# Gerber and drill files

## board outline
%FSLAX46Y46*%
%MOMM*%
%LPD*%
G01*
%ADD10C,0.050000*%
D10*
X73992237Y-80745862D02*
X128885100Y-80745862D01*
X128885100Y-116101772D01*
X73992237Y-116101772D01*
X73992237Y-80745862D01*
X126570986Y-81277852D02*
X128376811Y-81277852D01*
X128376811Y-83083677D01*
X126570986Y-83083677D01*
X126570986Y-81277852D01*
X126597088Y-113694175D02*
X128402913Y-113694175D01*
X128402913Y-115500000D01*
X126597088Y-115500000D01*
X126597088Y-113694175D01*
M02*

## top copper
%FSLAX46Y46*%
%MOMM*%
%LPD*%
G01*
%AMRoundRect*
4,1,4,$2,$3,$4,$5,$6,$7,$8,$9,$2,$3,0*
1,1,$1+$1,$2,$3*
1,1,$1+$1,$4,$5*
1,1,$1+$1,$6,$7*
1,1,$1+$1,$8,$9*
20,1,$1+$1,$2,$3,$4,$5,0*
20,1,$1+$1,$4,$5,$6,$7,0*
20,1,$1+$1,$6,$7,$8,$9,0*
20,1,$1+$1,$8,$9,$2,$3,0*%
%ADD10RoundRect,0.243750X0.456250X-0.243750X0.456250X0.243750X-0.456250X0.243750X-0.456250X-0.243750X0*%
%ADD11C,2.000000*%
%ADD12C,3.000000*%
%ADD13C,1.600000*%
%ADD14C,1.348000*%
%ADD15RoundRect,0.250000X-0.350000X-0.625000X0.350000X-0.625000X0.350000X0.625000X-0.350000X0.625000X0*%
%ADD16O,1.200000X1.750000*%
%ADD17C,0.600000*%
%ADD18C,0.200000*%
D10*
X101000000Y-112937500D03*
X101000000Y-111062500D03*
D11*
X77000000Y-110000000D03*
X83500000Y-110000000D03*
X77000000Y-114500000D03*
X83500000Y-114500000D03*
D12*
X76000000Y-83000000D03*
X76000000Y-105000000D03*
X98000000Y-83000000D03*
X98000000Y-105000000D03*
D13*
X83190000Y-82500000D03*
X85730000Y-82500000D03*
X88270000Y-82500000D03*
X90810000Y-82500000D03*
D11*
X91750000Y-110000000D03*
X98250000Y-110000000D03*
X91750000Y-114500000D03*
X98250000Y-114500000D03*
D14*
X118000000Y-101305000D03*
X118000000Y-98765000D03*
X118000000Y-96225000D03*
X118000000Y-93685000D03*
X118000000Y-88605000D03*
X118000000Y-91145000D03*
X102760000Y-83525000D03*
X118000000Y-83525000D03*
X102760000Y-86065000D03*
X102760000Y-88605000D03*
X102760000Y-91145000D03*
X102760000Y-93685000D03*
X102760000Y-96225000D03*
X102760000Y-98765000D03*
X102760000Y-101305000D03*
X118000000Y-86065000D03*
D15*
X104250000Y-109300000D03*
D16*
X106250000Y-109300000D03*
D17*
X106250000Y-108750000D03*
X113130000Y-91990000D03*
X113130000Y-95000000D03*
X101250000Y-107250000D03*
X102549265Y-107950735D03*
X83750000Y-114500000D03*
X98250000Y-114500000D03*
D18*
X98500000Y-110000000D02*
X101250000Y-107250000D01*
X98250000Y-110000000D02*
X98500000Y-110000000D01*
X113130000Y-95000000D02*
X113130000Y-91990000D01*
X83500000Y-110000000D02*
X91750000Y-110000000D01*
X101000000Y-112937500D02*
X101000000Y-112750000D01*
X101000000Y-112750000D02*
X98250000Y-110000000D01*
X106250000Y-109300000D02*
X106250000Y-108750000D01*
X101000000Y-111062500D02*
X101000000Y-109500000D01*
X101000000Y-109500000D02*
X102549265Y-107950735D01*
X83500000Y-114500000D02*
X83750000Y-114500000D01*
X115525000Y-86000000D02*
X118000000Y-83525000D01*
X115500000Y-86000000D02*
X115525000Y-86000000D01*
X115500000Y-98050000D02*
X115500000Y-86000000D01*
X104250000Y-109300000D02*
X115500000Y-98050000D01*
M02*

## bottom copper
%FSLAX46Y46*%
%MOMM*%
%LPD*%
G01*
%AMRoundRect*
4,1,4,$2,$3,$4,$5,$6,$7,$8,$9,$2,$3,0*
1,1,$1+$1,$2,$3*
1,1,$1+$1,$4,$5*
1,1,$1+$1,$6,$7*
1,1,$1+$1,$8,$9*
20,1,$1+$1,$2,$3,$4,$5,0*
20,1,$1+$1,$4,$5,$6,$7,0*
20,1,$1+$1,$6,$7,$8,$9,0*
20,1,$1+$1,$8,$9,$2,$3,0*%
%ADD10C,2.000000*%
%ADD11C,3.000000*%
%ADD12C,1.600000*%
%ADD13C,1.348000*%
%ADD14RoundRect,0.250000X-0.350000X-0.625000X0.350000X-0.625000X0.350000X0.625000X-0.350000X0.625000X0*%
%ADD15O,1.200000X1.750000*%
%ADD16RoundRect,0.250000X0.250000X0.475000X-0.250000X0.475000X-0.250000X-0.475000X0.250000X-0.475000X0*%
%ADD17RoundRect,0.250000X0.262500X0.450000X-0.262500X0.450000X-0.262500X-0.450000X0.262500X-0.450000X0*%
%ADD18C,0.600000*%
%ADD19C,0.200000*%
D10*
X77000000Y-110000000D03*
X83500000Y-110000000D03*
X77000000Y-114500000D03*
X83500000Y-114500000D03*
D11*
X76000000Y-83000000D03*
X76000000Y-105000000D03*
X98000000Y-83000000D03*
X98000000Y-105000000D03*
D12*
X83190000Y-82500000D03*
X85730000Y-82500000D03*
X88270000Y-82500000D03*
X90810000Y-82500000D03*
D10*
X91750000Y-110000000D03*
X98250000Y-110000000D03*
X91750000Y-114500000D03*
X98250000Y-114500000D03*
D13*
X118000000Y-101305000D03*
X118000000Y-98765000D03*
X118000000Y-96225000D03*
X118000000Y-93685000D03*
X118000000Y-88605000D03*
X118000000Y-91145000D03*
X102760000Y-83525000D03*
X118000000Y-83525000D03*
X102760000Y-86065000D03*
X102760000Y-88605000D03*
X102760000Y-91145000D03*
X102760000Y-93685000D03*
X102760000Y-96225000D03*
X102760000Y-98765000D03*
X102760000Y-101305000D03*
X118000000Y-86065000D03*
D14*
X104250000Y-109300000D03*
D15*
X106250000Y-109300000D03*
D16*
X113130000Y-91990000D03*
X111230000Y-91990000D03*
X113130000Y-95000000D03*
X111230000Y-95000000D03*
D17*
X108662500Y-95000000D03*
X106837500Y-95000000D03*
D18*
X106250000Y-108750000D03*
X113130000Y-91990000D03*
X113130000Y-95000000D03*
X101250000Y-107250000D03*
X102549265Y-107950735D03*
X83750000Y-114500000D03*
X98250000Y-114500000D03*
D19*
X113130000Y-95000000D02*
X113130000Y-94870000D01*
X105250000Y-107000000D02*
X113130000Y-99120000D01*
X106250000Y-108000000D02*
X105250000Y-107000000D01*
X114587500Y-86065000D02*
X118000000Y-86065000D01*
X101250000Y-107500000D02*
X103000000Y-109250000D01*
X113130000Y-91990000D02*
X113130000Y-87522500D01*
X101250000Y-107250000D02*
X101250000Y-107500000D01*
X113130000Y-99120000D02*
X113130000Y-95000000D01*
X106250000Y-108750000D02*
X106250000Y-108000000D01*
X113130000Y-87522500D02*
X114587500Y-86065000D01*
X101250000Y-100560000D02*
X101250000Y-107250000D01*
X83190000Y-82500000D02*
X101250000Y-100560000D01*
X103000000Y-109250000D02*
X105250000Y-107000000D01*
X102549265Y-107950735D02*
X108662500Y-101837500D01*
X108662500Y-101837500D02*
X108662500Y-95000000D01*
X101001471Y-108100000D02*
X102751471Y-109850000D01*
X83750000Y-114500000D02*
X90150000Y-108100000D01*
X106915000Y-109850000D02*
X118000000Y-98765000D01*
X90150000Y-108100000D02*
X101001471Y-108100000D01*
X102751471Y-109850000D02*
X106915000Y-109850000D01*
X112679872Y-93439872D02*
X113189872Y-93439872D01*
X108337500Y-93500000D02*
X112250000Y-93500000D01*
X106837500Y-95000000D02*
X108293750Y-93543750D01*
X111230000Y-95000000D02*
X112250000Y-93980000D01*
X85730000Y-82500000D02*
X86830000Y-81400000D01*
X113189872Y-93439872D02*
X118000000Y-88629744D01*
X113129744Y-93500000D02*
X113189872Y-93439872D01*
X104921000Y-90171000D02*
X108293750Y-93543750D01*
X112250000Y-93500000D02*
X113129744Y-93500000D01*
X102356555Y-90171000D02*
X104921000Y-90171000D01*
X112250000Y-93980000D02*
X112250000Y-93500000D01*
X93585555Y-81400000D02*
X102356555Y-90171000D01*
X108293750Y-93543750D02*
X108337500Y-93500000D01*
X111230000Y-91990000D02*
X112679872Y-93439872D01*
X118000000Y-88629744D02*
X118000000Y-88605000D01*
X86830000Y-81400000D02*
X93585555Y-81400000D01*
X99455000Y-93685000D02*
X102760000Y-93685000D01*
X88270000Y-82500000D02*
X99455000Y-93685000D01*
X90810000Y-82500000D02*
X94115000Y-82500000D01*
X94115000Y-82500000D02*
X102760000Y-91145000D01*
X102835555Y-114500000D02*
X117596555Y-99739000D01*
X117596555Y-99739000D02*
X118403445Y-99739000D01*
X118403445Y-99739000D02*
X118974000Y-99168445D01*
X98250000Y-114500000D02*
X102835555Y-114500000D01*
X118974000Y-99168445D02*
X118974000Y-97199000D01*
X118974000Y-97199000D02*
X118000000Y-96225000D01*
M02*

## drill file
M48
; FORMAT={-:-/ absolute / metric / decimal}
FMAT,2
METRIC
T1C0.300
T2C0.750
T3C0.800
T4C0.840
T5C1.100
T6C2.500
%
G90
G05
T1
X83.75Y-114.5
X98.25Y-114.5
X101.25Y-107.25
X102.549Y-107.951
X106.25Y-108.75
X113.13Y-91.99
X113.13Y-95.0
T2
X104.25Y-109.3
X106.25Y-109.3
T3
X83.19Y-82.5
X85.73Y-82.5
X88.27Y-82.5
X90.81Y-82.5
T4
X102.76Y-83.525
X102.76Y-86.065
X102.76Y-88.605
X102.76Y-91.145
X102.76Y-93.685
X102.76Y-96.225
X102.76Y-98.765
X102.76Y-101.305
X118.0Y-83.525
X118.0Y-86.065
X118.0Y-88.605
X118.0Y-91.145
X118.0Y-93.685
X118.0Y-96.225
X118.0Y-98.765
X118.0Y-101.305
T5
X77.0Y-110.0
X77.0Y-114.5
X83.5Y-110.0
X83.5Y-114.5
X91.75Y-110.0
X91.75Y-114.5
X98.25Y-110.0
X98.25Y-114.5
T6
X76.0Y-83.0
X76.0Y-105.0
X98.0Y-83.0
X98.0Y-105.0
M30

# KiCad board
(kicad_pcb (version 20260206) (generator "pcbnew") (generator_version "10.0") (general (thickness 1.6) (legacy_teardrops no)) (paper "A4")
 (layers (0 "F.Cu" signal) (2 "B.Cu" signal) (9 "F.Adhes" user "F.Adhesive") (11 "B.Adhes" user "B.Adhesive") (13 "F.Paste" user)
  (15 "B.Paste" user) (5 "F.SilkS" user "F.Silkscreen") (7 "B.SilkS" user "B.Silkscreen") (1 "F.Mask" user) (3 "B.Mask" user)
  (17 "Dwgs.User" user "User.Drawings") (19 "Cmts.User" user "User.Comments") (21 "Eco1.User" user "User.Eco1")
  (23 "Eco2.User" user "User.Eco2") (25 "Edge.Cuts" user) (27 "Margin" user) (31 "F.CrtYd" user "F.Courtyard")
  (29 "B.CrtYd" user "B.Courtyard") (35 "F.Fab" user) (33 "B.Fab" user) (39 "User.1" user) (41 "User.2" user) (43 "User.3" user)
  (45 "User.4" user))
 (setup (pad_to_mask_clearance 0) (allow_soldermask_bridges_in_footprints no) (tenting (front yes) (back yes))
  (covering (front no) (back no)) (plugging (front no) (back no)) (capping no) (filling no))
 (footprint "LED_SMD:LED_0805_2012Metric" (layer "F.Cu") (at 101 112 90)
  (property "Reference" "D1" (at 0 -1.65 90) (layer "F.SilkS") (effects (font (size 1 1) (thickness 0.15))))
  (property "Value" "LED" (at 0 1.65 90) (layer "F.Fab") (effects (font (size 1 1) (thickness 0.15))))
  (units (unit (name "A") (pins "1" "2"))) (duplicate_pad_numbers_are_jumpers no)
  (pad "1" smd roundrect (at -0.9375 0 90) (size 0.975 1.4) (layers "F.Cu" "F.Mask" "F.Paste") (roundrect_rratio 0.25) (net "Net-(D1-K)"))
  (pad "2" smd roundrect (at 0.9375 0 90) (size 0.975 1.4) (layers "F.Cu" "F.Mask" "F.Paste") (roundrect_rratio 0.25) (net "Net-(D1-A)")))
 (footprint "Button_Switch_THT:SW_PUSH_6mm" (layer "F.Cu") (at 77 110)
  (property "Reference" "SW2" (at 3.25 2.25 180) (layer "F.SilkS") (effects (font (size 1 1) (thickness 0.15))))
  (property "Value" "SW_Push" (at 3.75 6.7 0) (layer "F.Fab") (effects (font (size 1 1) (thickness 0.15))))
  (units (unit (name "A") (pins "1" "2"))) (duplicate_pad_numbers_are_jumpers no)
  (pad "1" thru_hole circle (at 0 0 90) (size 2 2) (drill 1.1) (layers "*.Cu" "*.Mask") (remove_unused_layers no) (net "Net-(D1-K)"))
  (pad "1" thru_hole circle (at 6.5 0 90) (size 2 2) (drill 1.1) (layers "*.Cu" "*.Mask") (remove_unused_layers no) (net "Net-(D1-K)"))
  (pad "2" thru_hole circle (at 0 4.5 90) (size 2 2) (drill 1.1) (layers "*.Cu" "*.Mask") (remove_unused_layers no) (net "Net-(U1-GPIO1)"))
  (pad "2" thru_hole circle (at 6.5 4.5 90) (size 2 2) (drill 1.1) (layers "*.Cu" "*.Mask") (remove_unused_layers no) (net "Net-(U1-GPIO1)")))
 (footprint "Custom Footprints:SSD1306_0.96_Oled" (layer "F.Cu") (at 74 107)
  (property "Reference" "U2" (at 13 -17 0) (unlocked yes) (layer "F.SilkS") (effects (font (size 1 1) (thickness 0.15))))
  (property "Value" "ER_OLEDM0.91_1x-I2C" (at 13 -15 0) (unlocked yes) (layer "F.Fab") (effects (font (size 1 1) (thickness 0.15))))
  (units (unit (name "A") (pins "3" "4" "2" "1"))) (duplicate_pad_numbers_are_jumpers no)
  (pad "" np_thru_hole circle (at 2 -24) (size 3 3) (drill 2.5) (layers "*.Cu" "*.Mask"))
  (pad "" np_thru_hole circle (at 2 -2) (size 3 3) (drill 2.5) (layers "*.Cu" "*.Mask"))
  (pad "" np_thru_hole circle (at 24 -24) (size 3 3) (drill 2.5) (layers "*.Cu" "*.Mask"))
  (pad "" np_thru_hole circle (at 24 -2) (size 3 3) (drill 2.5) (layers "*.Cu" "*.Mask"))
  (pad "1" thru_hole circle (at 9.19 -24.5) (size 1.6 1.6) (drill 0.8) (layers "*.Cu" "*.Mask") (remove_unused_layers no) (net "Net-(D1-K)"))
  (pad "2" thru_hole circle (at 11.73 -24.5) (size 1.6 1.6) (drill 0.8) (layers "*.Cu" "*.Mask") (remove_unused_layers no)
   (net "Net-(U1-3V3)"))
  (pad "3" thru_hole circle (at 14.27 -24.5) (size 1.6 1.6) (drill 0.8) (layers "*.Cu" "*.Mask") (remove_unused_layers no)
   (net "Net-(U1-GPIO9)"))
  (pad "4" thru_hole circle (at 16.81 -24.5) (size 1.6 1.6) (drill 0.8) (layers "*.Cu" "*.Mask") (remove_unused_layers no)
   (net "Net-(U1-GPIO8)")))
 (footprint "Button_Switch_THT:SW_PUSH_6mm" (layer "F.Cu") (at 91.75 110)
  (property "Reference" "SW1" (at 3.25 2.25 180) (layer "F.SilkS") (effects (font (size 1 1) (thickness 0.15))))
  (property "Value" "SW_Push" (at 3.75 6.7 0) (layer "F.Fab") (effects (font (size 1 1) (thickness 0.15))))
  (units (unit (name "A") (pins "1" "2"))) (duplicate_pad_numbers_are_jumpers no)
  (pad "1" thru_hole circle (at 0 0 90) (size 2 2) (drill 1.1) (layers "*.Cu" "*.Mask") (remove_unused_layers no) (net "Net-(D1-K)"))
  (pad "1" thru_hole circle (at 6.5 0 90) (size 2 2) (drill 1.1) (layers "*.Cu" "*.Mask") (remove_unused_layers no) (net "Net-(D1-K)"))
  (pad "2" thru_hole circle (at 0 4.5 90) (size 2 2) (drill 1.1) (layers "*.Cu" "*.Mask") (remove_unused_layers no) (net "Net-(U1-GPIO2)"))
  (pad "2" thru_hole circle (at 6.5 4.5 90) (size 2 2) (drill 1.1) (layers "*.Cu" "*.Mask") (remove_unused_layers no) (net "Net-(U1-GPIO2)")))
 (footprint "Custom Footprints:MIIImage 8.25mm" (layer "F.Cu") (at 124 88.25)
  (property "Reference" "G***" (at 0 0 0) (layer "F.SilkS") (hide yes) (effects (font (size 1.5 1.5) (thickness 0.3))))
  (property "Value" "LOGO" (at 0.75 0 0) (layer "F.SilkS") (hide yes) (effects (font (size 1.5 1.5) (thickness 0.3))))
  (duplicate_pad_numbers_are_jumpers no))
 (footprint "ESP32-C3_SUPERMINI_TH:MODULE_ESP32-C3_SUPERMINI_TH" (layer "F.Cu") (at 110.38 93.425)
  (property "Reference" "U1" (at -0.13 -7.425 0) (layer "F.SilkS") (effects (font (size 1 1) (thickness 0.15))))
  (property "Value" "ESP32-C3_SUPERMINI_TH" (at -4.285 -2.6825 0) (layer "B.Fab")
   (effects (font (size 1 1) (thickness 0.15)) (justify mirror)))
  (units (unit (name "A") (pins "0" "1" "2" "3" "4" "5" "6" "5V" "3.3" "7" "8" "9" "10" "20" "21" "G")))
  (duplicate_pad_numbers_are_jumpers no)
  (pad "0" thru_hole circle (at 7.62 7.88) (size 1.348 1.348) (drill 0.84) (layers "*.Cu" "*.Mask") (remove_unused_layers no)
   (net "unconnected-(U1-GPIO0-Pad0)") (solder_mask_margin 0.102))
  (pad "1" thru_hole circle (at 7.62 5.34) (size 1.348 1.348) (drill 0.84) (layers "*.Cu" "*.Mask") (remove_unused_layers no)
   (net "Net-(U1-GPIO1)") (solder_mask_margin 0.102))
  (pad "2" thru_hole circle (at 7.62 2.8) (size 1.348 1.348) (drill 0.84) (layers "*.Cu" "*.Mask") (remove_unused_layers no)
   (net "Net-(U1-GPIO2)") (solder_mask_margin 0.102))
  (pad "3" thru_hole circle (at 7.62 0.26) (size 1.348 1.348) (drill 0.84) (layers "*.Cu" "*.Mask") (remove_unused_layers no)
   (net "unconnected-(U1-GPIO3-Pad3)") (solder_mask_margin 0.102))
  (pad "3.3" thru_hole circle (at 7.62 -4.82) (size 1.348 1.348) (drill 0.84) (layers "*.Cu" "*.Mask") (remove_unused_layers no)
   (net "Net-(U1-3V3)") (solder_mask_margin 0.102))
  (pad "4" thru_hole circle (at 7.62 -2.28) (size 1.348 1.348) (drill 0.84) (layers "*.Cu" "*.Mask") (remove_unused_layers no)
   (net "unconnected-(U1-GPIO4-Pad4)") (solder_mask_margin 0.102))
  (pad "5" thru_hole circle (at -7.62 -9.9) (size 1.348 1.348) (drill 0.84) (layers "*.Cu" "*.Mask") (remove_unused_layers no)
   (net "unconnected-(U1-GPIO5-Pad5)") (solder_mask_margin 0.102))
  (pad "5V" thru_hole circle (at 7.62 -9.9) (size 1.348 1.348) (drill 0.84) (layers "*.Cu" "*.Mask") (remove_unused_layers no)
   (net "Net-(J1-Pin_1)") (solder_mask_margin 0.102))
  (pad "6" thru_hole circle (at -7.62 -7.36) (size 1.348 1.348) (drill 0.84) (layers "*.Cu" "*.Mask") (remove_unused_layers no)
   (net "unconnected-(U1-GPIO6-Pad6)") (solder_mask_margin 0.102))
  (pad "7" thru_hole circle (at -7.62 -4.82) (size 1.348 1.348) (drill 0.84) (layers "*.Cu" "*.Mask") (remove_unused_layers no)
   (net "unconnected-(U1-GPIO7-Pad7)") (solder_mask_margin 0.102))
  (pad "8" thru_hole circle (at -7.62 -2.28) (size 1.348 1.348) (drill 0.84) (layers "*.Cu" "*.Mask") (remove_unused_layers no)
   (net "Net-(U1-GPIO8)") (solder_mask_margin 0.102))
  (pad "9" thru_hole circle (at -7.62 0.26) (size 1.348 1.348) (drill 0.84) (layers "*.Cu" "*.Mask") (remove_unused_layers no)
   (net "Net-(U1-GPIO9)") (solder_mask_margin 0.102))
  (pad "10" thru_hole circle (at -7.62 2.8) (size 1.348 1.348) (drill 0.84) (layers "*.Cu" "*.Mask") (remove_unused_layers no)
   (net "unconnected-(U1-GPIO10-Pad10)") (solder_mask_margin 0.102))
  (pad "20" thru_hole circle (at -7.62 5.34) (size 1.348 1.348) (drill 0.84) (layers "*.Cu" "*.Mask") (remove_unused_layers no)
   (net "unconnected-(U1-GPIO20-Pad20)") (solder_mask_margin 0.102))
  (pad "21" thru_hole circle (at -7.62 7.88) (size 1.348 1.348) (drill 0.84) (layers "*.Cu" "*.Mask") (remove_unused_layers no)
   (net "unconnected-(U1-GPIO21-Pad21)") (solder_mask_margin 0.102))
  (pad "G" thru_hole circle (at 7.62 -7.36) (size 1.348 1.348) (drill 0.84) (layers "*.Cu" "*.Mask") (remove_unused_layers no)
   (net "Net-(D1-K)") (solder_mask_margin 0.102)))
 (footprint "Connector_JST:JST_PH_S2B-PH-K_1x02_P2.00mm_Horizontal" (layer "F.Cu") (at 104.25 109.3)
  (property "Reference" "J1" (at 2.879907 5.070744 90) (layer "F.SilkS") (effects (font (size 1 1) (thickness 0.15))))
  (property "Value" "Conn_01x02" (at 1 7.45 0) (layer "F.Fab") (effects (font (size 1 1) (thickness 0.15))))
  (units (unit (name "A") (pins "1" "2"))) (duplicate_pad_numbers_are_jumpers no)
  (pad "1" thru_hole roundrect (at 0 0) (size 1.2 1.75) (drill 0.75) (layers "*.Cu" "*.Mask") (remove_unused_layers no)
   (roundrect_rratio 0.208333) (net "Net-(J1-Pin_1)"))
  (pad "2" thru_hole oval (at 2 0) (size 1.2 1.75) (drill 0.75) (layers "*.Cu" "*.Mask") (remove_unused_layers no) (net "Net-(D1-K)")))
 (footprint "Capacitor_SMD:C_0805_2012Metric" (layer "B.Cu") (at 112.18 91.99 180)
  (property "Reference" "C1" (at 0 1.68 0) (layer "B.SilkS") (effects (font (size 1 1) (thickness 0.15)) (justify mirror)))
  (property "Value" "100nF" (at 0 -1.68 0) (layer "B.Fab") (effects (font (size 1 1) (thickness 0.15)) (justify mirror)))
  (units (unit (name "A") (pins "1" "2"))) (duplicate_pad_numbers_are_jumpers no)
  (pad "1" smd roundrect (at -0.95 0 180) (size 1 1.45) (layers "B.Cu" "B.Mask" "B.Paste") (roundrect_rratio 0.25) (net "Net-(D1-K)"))
  (pad "2" smd roundrect (at 0.95 0 180) (size 1 1.45) (layers "B.Cu" "B.Mask" "B.Paste") (roundrect_rratio 0.25) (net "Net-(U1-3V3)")))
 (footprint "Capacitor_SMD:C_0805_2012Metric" (layer "B.Cu") (at 112.18 95 180)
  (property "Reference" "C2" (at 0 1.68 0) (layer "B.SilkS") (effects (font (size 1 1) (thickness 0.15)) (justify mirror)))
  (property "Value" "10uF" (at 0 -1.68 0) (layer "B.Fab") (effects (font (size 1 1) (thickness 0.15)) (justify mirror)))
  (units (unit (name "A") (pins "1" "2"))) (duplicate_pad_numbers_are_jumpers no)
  (pad "1" smd roundrect (at -0.95 0 180) (size 1 1.45) (layers "B.Cu" "B.Mask" "B.Paste") (roundrect_rratio 0.25) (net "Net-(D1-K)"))
  (pad "2" smd roundrect (at 0.95 0 180) (size 1 1.45) (layers "B.Cu" "B.Mask" "B.Paste") (roundrect_rratio 0.25) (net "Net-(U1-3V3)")))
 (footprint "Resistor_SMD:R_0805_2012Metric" (layer "B.Cu") (at 107.75 95 180)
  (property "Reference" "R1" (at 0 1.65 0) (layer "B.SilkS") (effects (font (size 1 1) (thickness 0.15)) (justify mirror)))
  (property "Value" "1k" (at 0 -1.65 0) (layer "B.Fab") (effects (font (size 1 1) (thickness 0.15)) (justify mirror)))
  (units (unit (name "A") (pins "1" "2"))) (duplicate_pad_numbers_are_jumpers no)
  (pad "1" smd roundrect (at -0.9125 0 180) (size 1.025 1.4) (layers "B.Cu" "B.Mask" "B.Paste") (roundrect_rratio 0.243902)
   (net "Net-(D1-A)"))
  (pad "2" smd roundrect (at 0.9125 0 180) (size 1.025 1.4) (layers "B.Cu" "B.Mask" "B.Paste") (roundrect_rratio 0.243902)
   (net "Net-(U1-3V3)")))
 (gr_rect (start 73.992237 80.745862) (end 128.8851 116.101772) (stroke (width 0.05) (type default)) (fill no) (layer "Edge.Cuts"))
 (gr_rect (start 126.570986 81.277852) (end 128.376811 83.083677) (stroke (width 0.05) (type default)) (fill no) (layer "Edge.Cuts"))
 (gr_rect (start 126.597088 113.694175) (end 128.402913 115.5) (stroke (width 0.05) (type default)) (fill no) (layer "Edge.Cuts"))
 (segment (start 98.5 110) (end 101.25 107.25) (width 0.2) (layer "F.Cu") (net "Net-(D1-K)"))
 (segment (start 98.25 110) (end 98.5 110) (width 0.2) (layer "F.Cu") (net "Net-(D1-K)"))
 (segment (start 113.13 95) (end 113.13 91.99) (width 0.2) (layer "F.Cu") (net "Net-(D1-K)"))
 (segment (start 83.5 110) (end 91.75 110) (width 0.2) (layer "F.Cu") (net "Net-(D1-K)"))
 (segment (start 101 112.9375) (end 101 112.75) (width 0.2) (layer "F.Cu") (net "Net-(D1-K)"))
 (segment (start 101 112.75) (end 98.25 110) (width 0.2) (layer "F.Cu") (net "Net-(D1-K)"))
 (segment (start 106.25 109.3) (end 106.25 108.75) (width 0.2) (layer "F.Cu") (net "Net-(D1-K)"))
 (via (at 106.25 108.75) (size 0.6) (drill 0.3) (layers "F.Cu" "B.Cu") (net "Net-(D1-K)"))
 (via (at 113.13 91.99) (size 0.6) (drill 0.3) (layers "F.Cu" "B.Cu") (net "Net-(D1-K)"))
 (via (at 113.13 95) (size 0.6) (drill 0.3) (layers "F.Cu" "B.Cu") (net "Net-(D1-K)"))
 (via (at 101.25 107.25) (size 0.6) (drill 0.3) (layers "F.Cu" "B.Cu") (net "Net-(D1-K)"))
 (segment (start 113.13 95) (end 113.13 94.87) (width 0.2) (layer "B.Cu") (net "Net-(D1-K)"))
 (segment (start 105.25 107) (end 113.13 99.12) (width 0.2) (layer "B.Cu") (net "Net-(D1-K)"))
 (segment (start 106.25 108) (end 105.25 107) (width 0.2) (layer "B.Cu") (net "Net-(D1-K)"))
 (segment (start 114.5875 86.065) (end 118 86.065) (width 0.2) (layer "B.Cu") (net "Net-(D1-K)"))
 (segment (start 101.25 107.5) (end 103 109.25) (width 0.2) (layer "B.Cu") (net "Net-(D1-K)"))
 (segment (start 113.13 91.99) (end 113.13 87.5225) (width 0.2) (layer "B.Cu") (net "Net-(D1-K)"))
 (segment (start 101.25 107.25) (end 101.25 107.5) (width 0.2) (layer "B.Cu") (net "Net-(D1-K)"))
 (segment (start 113.13 99.12) (end 113.13 95) (width 0.2) (layer "B.Cu") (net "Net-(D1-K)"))
 (segment (start 106.25 108.75) (end 106.25 108) (width 0.2) (layer "B.Cu") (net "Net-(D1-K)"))
 (segment (start 113.13 87.5225) (end 114.5875 86.065) (width 0.2) (layer "B.Cu") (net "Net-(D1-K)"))
 (segment (start 101.25 100.56) (end 101.25 107.25) (width 0.2) (layer "B.Cu") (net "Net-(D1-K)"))
 (segment (start 83.19 82.5) (end 101.25 100.56) (width 0.2) (layer "B.Cu") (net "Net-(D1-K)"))
 (segment (start 103 109.25) (end 105.25 107) (width 0.2) (layer "B.Cu") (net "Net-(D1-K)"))
 (segment (start 101 111.0625) (end 101 109.5) (width 0.2) (layer "F.Cu") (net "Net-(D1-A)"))
 (segment (start 101 109.5) (end 102.549265 107.950735) (width 0.2) (layer "F.Cu") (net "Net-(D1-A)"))
 (via (at 102.549265 107.950735) (size 0.6) (drill 0.3) (layers "F.Cu" "B.Cu") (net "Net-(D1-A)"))
 (segment (start 102.549265 107.950735) (end 108.6625 101.8375) (width 0.2) (layer "B.Cu") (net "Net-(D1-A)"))
 (segment (start 108.6625 101.8375) (end 108.6625 95) (width 0.2) (layer "B.Cu") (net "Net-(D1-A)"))
 (segment (start 83.5 114.5) (end 83.75 114.5) (width 0.2) (layer "F.Cu") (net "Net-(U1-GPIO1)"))
 (via (at 83.75 114.5) (size 0.6) (drill 0.3) (layers "F.Cu" "B.Cu") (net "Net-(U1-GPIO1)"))
 (segment (start 101.001471 108.1) (end 102.751471 109.85) (width 0.2) (layer "B.Cu") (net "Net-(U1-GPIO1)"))
 (segment (start 83.75 114.5) (end 90.15 108.1) (width 0.2) (layer "B.Cu") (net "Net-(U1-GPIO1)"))
 (segment (start 106.915 109.85) (end 118 98.765) (width 0.2) (layer "B.Cu") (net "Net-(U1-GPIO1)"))
 (segment (start 90.15 108.1) (end 101.001471 108.1) (width 0.2) (layer "B.Cu") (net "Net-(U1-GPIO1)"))
 (segment (start 102.751471 109.85) (end 106.915 109.85) (width 0.2) (layer "B.Cu") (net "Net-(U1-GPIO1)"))
 (segment (start 112.679872 93.439872) (end 113.189872 93.439872) (width 0.2) (layer "B.Cu") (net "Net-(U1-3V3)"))
 (segment (start 108.3375 93.5) (end 112.25 93.5) (width 0.2) (layer "B.Cu") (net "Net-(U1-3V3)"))
 (segment (start 106.8375 95) (end 108.29375 93.54375) (width 0.2) (layer "B.Cu") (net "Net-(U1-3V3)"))
 (segment (start 111.23 95) (end 112.25 93.98) (width 0.2) (layer "B.Cu") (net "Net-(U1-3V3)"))
 (segment (start 85.73 82.5) (end 86.83 81.4) (width 0.2) (layer "B.Cu") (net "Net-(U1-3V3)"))
 (segment (start 113.189872 93.439872) (end 118 88.629744) (width 0.2) (layer "B.Cu") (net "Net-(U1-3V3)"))
 (segment (start 113.129744 93.5) (end 113.189872 93.439872) (width 0.2) (layer "B.Cu") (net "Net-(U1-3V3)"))
 (segment (start 104.921 90.171) (end 108.29375 93.54375) (width 0.2) (layer "B.Cu") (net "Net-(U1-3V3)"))
 (segment (start 112.25 93.5) (end 113.129744 93.5) (width 0.2) (layer "B.Cu") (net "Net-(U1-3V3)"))
 (segment (start 102.356555 90.171) (end 104.921 90.171) (width 0.2) (layer "B.Cu") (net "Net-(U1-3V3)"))
 (segment (start 112.25 93.98) (end 112.25 93.5) (width 0.2) (layer "B.Cu") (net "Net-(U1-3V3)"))
 (segment (start 93.585555 81.4) (end 102.356555 90.171) (width 0.2) (layer "B.Cu") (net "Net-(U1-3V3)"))
 (segment (start 108.29375 93.54375) (end 108.3375 93.5) (width 0.2) (layer "B.Cu") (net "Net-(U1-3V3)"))
 (segment (start 111.23 91.99) (end 112.679872 93.439872) (width 0.2) (layer "B.Cu") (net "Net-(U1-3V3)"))
 (segment (start 118 88.629744) (end 118 88.605) (width 0.2) (layer "B.Cu") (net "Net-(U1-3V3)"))
 (segment (start 86.83 81.4) (end 93.585555 81.4) (width 0.2) (layer "B.Cu") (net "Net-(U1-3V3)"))
 (segment (start 99.455 93.685) (end 102.76 93.685) (width 0.2) (layer "B.Cu") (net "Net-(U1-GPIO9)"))
 (segment (start 88.27 82.5) (end 99.455 93.685) (width 0.2) (layer "B.Cu") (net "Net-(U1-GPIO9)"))
 (segment (start 90.81 82.5) (end 94.115 82.5) (width 0.2) (layer "B.Cu") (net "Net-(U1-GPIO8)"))
 (segment (start 94.115 82.5) (end 102.76 91.145) (width 0.2) (layer "B.Cu") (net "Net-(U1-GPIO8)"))
 (via (at 98.25 114.5) (size 0.6) (drill 0.3) (layers "F.Cu" "B.Cu") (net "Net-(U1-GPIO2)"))
 (segment (start 102.835555 114.5) (end 117.596555 99.739) (width 0.2) (layer "B.Cu") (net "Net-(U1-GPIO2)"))
 (segment (start 117.596555 99.739) (end 118.403445 99.739) (width 0.2) (layer "B.Cu") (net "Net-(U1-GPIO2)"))
 (segment (start 118.403445 99.739) (end 118.974 99.168445) (width 0.2) (layer "B.Cu") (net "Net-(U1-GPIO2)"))
 (segment (start 98.25 114.5) (end 102.835555 114.5) (width 0.2) (layer "B.Cu") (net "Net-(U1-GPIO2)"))
 (segment (start 118.974 99.168445) (end 118.974 97.199) (width 0.2) (layer "B.Cu") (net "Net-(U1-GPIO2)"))
 (segment (start 118.974 97.199) (end 118 96.225) (width 0.2) (layer "B.Cu") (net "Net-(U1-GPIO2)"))
 (segment (start 115.525 86) (end 118 83.525) (width 0.2) (layer "F.Cu") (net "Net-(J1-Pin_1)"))
 (segment (start 115.5 86) (end 115.525 86) (width 0.2) (layer "F.Cu") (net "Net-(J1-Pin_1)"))
 (segment (start 115.5 98.05) (end 115.5 86) (width 0.2) (layer "F.Cu") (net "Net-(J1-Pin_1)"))
 (segment (start 104.25 109.3) (end 115.5 98.05) (width 0.2) (layer "F.Cu") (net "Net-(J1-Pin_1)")))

